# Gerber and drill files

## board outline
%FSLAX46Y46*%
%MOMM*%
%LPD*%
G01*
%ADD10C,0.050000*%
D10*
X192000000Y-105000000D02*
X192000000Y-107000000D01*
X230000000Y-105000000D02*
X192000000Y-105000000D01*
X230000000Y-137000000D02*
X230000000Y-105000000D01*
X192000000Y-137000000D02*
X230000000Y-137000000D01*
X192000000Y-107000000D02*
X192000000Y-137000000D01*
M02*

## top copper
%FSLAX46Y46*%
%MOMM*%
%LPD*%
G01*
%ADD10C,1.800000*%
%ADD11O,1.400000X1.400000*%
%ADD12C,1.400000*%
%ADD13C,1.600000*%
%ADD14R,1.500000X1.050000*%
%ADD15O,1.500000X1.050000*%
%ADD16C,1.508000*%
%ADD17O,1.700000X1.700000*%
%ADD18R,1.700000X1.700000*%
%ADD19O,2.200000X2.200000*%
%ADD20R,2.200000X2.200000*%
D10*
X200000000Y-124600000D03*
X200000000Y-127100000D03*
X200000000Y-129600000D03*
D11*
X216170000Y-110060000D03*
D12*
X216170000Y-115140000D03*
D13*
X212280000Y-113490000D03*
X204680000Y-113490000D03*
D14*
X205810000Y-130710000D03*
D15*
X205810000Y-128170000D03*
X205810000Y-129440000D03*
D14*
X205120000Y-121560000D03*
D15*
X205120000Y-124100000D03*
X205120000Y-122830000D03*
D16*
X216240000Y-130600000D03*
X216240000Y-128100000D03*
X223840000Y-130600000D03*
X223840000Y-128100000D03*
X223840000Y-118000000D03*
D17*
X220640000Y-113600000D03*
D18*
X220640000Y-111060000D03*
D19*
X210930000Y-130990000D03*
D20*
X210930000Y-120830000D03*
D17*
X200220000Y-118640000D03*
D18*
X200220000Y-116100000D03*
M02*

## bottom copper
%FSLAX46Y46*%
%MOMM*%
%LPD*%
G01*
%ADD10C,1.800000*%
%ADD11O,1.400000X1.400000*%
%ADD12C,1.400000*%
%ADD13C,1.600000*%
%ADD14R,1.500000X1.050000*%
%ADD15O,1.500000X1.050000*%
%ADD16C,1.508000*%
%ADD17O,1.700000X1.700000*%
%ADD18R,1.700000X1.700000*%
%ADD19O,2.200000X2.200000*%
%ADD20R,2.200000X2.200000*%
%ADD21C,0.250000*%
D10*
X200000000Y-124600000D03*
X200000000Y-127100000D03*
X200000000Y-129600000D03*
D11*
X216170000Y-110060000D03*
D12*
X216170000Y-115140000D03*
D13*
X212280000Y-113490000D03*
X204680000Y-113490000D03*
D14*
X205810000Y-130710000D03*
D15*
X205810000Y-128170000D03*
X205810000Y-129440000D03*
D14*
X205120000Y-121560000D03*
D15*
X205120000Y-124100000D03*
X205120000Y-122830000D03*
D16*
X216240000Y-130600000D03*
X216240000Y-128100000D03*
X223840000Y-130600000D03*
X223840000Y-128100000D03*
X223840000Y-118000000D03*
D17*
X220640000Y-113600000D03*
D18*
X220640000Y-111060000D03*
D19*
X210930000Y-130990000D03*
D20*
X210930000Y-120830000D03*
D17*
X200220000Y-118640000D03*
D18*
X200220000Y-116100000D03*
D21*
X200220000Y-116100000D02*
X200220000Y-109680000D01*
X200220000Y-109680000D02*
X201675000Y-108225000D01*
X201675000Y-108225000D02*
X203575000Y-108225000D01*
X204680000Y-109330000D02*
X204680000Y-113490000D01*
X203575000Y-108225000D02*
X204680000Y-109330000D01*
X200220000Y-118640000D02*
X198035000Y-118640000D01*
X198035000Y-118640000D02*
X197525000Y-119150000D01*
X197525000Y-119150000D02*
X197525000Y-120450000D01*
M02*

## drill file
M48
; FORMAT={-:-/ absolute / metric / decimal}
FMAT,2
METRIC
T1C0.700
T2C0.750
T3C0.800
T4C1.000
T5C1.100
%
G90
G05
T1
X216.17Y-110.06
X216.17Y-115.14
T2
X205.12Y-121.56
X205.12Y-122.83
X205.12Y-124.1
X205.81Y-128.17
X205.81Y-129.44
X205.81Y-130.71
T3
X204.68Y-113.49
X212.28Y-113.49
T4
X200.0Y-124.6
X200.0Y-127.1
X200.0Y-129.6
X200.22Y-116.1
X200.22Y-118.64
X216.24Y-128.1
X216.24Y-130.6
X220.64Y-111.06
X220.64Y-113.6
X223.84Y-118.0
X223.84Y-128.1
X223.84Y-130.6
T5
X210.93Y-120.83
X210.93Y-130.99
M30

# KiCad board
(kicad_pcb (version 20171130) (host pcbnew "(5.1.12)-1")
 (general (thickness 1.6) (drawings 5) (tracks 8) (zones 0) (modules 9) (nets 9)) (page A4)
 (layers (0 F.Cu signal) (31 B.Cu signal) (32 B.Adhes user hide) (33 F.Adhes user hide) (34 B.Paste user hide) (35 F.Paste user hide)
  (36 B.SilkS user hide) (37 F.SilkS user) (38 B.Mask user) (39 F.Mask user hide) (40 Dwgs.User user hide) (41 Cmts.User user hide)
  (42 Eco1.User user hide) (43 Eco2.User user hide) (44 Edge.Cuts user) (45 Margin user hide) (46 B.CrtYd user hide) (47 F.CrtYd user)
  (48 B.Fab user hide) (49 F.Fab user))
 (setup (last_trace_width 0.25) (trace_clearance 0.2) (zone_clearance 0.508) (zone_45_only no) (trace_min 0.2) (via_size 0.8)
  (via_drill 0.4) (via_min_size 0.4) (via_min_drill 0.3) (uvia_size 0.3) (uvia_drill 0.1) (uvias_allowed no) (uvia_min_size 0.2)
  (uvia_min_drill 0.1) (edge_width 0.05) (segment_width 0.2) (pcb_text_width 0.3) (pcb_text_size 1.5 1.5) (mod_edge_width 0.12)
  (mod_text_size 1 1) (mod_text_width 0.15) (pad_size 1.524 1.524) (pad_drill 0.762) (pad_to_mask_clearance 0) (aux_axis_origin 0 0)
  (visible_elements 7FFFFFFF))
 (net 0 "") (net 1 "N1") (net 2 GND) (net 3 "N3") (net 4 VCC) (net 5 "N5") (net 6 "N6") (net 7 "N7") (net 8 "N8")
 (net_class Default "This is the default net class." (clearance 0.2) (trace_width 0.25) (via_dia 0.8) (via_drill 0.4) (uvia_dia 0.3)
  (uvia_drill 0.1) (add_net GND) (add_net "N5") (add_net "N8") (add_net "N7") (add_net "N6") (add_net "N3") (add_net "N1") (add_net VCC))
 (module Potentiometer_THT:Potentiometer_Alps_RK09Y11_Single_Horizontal (layer F.Cu) (at 200 124.6 180)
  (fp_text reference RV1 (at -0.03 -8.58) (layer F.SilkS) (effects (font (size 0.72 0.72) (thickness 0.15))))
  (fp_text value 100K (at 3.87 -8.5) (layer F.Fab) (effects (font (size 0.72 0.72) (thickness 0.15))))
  (pad 1 thru_hole circle (at 0 0 180) (size 1.8 1.8) (drill 1) (layers *.Cu *.Mask) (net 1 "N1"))
  (pad 2 thru_hole circle (at 0 -2.5 180) (size 1.8 1.8) (drill 1) (layers *.Cu *.Mask) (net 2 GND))
  (pad 3 thru_hole circle (at 0 -5 180) (size 1.8 1.8) (drill 1) (layers *.Cu *.Mask) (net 2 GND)))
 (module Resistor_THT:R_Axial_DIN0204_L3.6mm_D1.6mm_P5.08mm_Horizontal (layer F.Cu) (at 216.17 115.14 90)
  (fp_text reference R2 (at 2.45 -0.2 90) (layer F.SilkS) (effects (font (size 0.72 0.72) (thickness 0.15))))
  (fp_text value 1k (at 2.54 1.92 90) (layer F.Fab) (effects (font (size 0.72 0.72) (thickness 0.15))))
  (pad 2 thru_hole oval (at 5.08 0 90) (size 1.4 1.4) (drill 0.7) (layers *.Cu *.Mask) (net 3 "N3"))
  (pad 1 thru_hole circle (at 0 0 90) (size 1.4 1.4) (drill 0.7) (layers *.Cu *.Mask) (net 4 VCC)))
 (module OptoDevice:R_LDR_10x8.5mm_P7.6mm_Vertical (layer F.Cu) (at 204.68 113.49)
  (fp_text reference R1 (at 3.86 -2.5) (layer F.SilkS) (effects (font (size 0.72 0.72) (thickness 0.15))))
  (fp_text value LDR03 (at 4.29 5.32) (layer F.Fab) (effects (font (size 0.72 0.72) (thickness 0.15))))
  (pad 2 thru_hole circle (at 7.6 0) (size 1.6 1.6) (drill 0.8) (layers *.Cu *.Mask) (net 1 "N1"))
  (pad 1 thru_hole circle (at 0 0) (size 1.6 1.6) (drill 0.8) (layers *.Cu *.Mask) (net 4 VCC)))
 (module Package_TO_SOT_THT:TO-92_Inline (layer F.Cu) (at 205.81 130.71 90)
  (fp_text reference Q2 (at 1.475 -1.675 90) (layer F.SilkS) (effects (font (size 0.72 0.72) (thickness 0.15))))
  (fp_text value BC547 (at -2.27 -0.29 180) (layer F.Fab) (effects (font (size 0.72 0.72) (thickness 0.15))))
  (pad 1 thru_hole rect (at 0 0 90) (size 1.05 1.5) (drill 0.75) (layers *.Cu *.Mask) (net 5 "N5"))
  (pad 3 thru_hole oval (at 2.54 0 90) (size 1.05 1.5) (drill 0.75) (layers *.Cu *.Mask) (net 2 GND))
  (pad 2 thru_hole oval (at 1.27 0 90) (size 1.05 1.5) (drill 0.75) (layers *.Cu *.Mask) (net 3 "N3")))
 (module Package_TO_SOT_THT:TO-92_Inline (layer F.Cu) (at 205.12 121.56 270)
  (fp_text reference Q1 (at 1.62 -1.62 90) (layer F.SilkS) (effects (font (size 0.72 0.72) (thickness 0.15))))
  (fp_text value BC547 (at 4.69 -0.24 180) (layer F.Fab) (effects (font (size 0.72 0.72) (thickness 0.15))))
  (pad 1 thru_hole rect (at 0 0 270) (size 1.05 1.5) (drill 0.75) (layers *.Cu *.Mask) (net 3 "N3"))
  (pad 3 thru_hole oval (at 2.54 0 270) (size 1.05 1.5) (drill 0.75) (layers *.Cu *.Mask) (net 2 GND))
  (pad 2 thru_hole oval (at 1.27 0 270) (size 1.05 1.5) (drill 0.75) (layers *.Cu *.Mask) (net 1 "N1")))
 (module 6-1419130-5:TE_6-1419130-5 (layer F.Cu) (at 220.04 124.3 90)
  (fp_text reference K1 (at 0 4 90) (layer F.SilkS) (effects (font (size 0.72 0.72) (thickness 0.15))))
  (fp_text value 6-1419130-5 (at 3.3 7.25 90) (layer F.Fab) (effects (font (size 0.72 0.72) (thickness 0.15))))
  (pad 12 thru_hole circle (at -6.3 -3.8 90) (size 1.508 1.508) (drill 1) (layers *.Cu *.Mask) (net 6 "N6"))
  (pad 14 thru_hole circle (at -3.8 -3.8 90) (size 1.508 1.508) (drill 1) (layers *.Cu *.Mask) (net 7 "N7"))
  (pad A1 thru_hole circle (at -6.3 3.8 90) (size 1.508 1.508) (drill 1) (layers *.Cu *.Mask) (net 5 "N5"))
  (pad A2 thru_hole circle (at -3.8 3.8 90) (size 1.508 1.508) (drill 1) (layers *.Cu *.Mask) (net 4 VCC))
  (pad 11 thru_hole circle (at 6.3 3.8 90) (size 1.508 1.508) (drill 1) (layers *.Cu *.Mask) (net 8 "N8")))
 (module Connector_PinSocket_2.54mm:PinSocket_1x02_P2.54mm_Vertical (layer F.Cu) (at 220.64 111.06)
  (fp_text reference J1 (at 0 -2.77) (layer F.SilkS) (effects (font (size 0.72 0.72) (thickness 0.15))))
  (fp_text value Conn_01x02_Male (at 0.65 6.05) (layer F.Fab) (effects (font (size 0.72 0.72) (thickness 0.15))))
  (pad 2 thru_hole oval (at 0 2.54) (size 1.7 1.7) (drill 1) (layers *.Cu *.Mask) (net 7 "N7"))
  (pad 1 thru_hole rect (at 0 0) (size 1.7 1.7) (drill 1) (layers *.Cu *.Mask) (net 8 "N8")))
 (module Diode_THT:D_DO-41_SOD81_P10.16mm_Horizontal (layer F.Cu) (at 210.93 120.83 270)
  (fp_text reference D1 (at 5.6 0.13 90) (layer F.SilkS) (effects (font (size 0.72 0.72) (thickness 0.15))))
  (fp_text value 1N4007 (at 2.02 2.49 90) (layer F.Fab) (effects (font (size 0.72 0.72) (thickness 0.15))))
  (pad 2 thru_hole oval (at 10.16 0 270) (size 2.2 2.2) (drill 1.1) (layers *.Cu *.Mask) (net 5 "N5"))
  (pad 1 thru_hole rect (at 0 0 270) (size 2.2 2.2) (drill 1.1) (layers *.Cu *.Mask) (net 4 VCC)))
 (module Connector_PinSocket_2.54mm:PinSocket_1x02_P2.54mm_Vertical (layer F.Cu) (at 200.22 116.1)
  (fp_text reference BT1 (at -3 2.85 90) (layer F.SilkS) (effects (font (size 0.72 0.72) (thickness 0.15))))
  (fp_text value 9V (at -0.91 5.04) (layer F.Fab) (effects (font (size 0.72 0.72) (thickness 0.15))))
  (pad 2 thru_hole oval (at 0 2.54) (size 1.7 1.7) (drill 1) (layers *.Cu *.Mask) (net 2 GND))
  (pad 1 thru_hole rect (at 0 0) (size 1.7 1.7) (drill 1) (layers *.Cu *.Mask) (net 4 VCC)))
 (gr_line (start 192 105) (end 192 107) (layer Edge.Cuts) (width 0.05))
 (gr_line (start 230 105) (end 192 105) (layer Edge.Cuts) (width 0.05))
 (gr_line (start 230 137) (end 230 105) (layer Edge.Cuts) (width 0.05))
 (gr_line (start 192 137) (end 230 137) (layer Edge.Cuts) (width 0.05))
 (gr_line (start 192 107) (end 192 137) (layer Edge.Cuts) (width 0.05))
 (segment (start 200.22 116.1) (end 200.22 109.68) (width 0.25) (layer B.Cu) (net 4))
 (segment (start 200.22 109.68) (end 201.675 108.225) (width 0.25) (layer B.Cu) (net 4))
 (segment (start 201.675 108.225) (end 203.575 108.225) (width 0.25) (layer B.Cu) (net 4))
 (segment (start 204.68 109.33) (end 204.68 113.49) (width 0.25) (layer B.Cu) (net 4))
 (segment (start 203.575 108.225) (end 204.68 109.33) (width 0.25) (layer B.Cu) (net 4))
 (segment (start 200.22 118.64) (end 198.035 118.64) (width 0.25) (layer B.Cu) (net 2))
 (segment (start 198.035 118.64) (end 197.525 119.15) (width 0.25) (layer B.Cu) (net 2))
 (segment (start 197.525 119.15) (end 197.525 120.45) (width 0.25) (layer B.Cu) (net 2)))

